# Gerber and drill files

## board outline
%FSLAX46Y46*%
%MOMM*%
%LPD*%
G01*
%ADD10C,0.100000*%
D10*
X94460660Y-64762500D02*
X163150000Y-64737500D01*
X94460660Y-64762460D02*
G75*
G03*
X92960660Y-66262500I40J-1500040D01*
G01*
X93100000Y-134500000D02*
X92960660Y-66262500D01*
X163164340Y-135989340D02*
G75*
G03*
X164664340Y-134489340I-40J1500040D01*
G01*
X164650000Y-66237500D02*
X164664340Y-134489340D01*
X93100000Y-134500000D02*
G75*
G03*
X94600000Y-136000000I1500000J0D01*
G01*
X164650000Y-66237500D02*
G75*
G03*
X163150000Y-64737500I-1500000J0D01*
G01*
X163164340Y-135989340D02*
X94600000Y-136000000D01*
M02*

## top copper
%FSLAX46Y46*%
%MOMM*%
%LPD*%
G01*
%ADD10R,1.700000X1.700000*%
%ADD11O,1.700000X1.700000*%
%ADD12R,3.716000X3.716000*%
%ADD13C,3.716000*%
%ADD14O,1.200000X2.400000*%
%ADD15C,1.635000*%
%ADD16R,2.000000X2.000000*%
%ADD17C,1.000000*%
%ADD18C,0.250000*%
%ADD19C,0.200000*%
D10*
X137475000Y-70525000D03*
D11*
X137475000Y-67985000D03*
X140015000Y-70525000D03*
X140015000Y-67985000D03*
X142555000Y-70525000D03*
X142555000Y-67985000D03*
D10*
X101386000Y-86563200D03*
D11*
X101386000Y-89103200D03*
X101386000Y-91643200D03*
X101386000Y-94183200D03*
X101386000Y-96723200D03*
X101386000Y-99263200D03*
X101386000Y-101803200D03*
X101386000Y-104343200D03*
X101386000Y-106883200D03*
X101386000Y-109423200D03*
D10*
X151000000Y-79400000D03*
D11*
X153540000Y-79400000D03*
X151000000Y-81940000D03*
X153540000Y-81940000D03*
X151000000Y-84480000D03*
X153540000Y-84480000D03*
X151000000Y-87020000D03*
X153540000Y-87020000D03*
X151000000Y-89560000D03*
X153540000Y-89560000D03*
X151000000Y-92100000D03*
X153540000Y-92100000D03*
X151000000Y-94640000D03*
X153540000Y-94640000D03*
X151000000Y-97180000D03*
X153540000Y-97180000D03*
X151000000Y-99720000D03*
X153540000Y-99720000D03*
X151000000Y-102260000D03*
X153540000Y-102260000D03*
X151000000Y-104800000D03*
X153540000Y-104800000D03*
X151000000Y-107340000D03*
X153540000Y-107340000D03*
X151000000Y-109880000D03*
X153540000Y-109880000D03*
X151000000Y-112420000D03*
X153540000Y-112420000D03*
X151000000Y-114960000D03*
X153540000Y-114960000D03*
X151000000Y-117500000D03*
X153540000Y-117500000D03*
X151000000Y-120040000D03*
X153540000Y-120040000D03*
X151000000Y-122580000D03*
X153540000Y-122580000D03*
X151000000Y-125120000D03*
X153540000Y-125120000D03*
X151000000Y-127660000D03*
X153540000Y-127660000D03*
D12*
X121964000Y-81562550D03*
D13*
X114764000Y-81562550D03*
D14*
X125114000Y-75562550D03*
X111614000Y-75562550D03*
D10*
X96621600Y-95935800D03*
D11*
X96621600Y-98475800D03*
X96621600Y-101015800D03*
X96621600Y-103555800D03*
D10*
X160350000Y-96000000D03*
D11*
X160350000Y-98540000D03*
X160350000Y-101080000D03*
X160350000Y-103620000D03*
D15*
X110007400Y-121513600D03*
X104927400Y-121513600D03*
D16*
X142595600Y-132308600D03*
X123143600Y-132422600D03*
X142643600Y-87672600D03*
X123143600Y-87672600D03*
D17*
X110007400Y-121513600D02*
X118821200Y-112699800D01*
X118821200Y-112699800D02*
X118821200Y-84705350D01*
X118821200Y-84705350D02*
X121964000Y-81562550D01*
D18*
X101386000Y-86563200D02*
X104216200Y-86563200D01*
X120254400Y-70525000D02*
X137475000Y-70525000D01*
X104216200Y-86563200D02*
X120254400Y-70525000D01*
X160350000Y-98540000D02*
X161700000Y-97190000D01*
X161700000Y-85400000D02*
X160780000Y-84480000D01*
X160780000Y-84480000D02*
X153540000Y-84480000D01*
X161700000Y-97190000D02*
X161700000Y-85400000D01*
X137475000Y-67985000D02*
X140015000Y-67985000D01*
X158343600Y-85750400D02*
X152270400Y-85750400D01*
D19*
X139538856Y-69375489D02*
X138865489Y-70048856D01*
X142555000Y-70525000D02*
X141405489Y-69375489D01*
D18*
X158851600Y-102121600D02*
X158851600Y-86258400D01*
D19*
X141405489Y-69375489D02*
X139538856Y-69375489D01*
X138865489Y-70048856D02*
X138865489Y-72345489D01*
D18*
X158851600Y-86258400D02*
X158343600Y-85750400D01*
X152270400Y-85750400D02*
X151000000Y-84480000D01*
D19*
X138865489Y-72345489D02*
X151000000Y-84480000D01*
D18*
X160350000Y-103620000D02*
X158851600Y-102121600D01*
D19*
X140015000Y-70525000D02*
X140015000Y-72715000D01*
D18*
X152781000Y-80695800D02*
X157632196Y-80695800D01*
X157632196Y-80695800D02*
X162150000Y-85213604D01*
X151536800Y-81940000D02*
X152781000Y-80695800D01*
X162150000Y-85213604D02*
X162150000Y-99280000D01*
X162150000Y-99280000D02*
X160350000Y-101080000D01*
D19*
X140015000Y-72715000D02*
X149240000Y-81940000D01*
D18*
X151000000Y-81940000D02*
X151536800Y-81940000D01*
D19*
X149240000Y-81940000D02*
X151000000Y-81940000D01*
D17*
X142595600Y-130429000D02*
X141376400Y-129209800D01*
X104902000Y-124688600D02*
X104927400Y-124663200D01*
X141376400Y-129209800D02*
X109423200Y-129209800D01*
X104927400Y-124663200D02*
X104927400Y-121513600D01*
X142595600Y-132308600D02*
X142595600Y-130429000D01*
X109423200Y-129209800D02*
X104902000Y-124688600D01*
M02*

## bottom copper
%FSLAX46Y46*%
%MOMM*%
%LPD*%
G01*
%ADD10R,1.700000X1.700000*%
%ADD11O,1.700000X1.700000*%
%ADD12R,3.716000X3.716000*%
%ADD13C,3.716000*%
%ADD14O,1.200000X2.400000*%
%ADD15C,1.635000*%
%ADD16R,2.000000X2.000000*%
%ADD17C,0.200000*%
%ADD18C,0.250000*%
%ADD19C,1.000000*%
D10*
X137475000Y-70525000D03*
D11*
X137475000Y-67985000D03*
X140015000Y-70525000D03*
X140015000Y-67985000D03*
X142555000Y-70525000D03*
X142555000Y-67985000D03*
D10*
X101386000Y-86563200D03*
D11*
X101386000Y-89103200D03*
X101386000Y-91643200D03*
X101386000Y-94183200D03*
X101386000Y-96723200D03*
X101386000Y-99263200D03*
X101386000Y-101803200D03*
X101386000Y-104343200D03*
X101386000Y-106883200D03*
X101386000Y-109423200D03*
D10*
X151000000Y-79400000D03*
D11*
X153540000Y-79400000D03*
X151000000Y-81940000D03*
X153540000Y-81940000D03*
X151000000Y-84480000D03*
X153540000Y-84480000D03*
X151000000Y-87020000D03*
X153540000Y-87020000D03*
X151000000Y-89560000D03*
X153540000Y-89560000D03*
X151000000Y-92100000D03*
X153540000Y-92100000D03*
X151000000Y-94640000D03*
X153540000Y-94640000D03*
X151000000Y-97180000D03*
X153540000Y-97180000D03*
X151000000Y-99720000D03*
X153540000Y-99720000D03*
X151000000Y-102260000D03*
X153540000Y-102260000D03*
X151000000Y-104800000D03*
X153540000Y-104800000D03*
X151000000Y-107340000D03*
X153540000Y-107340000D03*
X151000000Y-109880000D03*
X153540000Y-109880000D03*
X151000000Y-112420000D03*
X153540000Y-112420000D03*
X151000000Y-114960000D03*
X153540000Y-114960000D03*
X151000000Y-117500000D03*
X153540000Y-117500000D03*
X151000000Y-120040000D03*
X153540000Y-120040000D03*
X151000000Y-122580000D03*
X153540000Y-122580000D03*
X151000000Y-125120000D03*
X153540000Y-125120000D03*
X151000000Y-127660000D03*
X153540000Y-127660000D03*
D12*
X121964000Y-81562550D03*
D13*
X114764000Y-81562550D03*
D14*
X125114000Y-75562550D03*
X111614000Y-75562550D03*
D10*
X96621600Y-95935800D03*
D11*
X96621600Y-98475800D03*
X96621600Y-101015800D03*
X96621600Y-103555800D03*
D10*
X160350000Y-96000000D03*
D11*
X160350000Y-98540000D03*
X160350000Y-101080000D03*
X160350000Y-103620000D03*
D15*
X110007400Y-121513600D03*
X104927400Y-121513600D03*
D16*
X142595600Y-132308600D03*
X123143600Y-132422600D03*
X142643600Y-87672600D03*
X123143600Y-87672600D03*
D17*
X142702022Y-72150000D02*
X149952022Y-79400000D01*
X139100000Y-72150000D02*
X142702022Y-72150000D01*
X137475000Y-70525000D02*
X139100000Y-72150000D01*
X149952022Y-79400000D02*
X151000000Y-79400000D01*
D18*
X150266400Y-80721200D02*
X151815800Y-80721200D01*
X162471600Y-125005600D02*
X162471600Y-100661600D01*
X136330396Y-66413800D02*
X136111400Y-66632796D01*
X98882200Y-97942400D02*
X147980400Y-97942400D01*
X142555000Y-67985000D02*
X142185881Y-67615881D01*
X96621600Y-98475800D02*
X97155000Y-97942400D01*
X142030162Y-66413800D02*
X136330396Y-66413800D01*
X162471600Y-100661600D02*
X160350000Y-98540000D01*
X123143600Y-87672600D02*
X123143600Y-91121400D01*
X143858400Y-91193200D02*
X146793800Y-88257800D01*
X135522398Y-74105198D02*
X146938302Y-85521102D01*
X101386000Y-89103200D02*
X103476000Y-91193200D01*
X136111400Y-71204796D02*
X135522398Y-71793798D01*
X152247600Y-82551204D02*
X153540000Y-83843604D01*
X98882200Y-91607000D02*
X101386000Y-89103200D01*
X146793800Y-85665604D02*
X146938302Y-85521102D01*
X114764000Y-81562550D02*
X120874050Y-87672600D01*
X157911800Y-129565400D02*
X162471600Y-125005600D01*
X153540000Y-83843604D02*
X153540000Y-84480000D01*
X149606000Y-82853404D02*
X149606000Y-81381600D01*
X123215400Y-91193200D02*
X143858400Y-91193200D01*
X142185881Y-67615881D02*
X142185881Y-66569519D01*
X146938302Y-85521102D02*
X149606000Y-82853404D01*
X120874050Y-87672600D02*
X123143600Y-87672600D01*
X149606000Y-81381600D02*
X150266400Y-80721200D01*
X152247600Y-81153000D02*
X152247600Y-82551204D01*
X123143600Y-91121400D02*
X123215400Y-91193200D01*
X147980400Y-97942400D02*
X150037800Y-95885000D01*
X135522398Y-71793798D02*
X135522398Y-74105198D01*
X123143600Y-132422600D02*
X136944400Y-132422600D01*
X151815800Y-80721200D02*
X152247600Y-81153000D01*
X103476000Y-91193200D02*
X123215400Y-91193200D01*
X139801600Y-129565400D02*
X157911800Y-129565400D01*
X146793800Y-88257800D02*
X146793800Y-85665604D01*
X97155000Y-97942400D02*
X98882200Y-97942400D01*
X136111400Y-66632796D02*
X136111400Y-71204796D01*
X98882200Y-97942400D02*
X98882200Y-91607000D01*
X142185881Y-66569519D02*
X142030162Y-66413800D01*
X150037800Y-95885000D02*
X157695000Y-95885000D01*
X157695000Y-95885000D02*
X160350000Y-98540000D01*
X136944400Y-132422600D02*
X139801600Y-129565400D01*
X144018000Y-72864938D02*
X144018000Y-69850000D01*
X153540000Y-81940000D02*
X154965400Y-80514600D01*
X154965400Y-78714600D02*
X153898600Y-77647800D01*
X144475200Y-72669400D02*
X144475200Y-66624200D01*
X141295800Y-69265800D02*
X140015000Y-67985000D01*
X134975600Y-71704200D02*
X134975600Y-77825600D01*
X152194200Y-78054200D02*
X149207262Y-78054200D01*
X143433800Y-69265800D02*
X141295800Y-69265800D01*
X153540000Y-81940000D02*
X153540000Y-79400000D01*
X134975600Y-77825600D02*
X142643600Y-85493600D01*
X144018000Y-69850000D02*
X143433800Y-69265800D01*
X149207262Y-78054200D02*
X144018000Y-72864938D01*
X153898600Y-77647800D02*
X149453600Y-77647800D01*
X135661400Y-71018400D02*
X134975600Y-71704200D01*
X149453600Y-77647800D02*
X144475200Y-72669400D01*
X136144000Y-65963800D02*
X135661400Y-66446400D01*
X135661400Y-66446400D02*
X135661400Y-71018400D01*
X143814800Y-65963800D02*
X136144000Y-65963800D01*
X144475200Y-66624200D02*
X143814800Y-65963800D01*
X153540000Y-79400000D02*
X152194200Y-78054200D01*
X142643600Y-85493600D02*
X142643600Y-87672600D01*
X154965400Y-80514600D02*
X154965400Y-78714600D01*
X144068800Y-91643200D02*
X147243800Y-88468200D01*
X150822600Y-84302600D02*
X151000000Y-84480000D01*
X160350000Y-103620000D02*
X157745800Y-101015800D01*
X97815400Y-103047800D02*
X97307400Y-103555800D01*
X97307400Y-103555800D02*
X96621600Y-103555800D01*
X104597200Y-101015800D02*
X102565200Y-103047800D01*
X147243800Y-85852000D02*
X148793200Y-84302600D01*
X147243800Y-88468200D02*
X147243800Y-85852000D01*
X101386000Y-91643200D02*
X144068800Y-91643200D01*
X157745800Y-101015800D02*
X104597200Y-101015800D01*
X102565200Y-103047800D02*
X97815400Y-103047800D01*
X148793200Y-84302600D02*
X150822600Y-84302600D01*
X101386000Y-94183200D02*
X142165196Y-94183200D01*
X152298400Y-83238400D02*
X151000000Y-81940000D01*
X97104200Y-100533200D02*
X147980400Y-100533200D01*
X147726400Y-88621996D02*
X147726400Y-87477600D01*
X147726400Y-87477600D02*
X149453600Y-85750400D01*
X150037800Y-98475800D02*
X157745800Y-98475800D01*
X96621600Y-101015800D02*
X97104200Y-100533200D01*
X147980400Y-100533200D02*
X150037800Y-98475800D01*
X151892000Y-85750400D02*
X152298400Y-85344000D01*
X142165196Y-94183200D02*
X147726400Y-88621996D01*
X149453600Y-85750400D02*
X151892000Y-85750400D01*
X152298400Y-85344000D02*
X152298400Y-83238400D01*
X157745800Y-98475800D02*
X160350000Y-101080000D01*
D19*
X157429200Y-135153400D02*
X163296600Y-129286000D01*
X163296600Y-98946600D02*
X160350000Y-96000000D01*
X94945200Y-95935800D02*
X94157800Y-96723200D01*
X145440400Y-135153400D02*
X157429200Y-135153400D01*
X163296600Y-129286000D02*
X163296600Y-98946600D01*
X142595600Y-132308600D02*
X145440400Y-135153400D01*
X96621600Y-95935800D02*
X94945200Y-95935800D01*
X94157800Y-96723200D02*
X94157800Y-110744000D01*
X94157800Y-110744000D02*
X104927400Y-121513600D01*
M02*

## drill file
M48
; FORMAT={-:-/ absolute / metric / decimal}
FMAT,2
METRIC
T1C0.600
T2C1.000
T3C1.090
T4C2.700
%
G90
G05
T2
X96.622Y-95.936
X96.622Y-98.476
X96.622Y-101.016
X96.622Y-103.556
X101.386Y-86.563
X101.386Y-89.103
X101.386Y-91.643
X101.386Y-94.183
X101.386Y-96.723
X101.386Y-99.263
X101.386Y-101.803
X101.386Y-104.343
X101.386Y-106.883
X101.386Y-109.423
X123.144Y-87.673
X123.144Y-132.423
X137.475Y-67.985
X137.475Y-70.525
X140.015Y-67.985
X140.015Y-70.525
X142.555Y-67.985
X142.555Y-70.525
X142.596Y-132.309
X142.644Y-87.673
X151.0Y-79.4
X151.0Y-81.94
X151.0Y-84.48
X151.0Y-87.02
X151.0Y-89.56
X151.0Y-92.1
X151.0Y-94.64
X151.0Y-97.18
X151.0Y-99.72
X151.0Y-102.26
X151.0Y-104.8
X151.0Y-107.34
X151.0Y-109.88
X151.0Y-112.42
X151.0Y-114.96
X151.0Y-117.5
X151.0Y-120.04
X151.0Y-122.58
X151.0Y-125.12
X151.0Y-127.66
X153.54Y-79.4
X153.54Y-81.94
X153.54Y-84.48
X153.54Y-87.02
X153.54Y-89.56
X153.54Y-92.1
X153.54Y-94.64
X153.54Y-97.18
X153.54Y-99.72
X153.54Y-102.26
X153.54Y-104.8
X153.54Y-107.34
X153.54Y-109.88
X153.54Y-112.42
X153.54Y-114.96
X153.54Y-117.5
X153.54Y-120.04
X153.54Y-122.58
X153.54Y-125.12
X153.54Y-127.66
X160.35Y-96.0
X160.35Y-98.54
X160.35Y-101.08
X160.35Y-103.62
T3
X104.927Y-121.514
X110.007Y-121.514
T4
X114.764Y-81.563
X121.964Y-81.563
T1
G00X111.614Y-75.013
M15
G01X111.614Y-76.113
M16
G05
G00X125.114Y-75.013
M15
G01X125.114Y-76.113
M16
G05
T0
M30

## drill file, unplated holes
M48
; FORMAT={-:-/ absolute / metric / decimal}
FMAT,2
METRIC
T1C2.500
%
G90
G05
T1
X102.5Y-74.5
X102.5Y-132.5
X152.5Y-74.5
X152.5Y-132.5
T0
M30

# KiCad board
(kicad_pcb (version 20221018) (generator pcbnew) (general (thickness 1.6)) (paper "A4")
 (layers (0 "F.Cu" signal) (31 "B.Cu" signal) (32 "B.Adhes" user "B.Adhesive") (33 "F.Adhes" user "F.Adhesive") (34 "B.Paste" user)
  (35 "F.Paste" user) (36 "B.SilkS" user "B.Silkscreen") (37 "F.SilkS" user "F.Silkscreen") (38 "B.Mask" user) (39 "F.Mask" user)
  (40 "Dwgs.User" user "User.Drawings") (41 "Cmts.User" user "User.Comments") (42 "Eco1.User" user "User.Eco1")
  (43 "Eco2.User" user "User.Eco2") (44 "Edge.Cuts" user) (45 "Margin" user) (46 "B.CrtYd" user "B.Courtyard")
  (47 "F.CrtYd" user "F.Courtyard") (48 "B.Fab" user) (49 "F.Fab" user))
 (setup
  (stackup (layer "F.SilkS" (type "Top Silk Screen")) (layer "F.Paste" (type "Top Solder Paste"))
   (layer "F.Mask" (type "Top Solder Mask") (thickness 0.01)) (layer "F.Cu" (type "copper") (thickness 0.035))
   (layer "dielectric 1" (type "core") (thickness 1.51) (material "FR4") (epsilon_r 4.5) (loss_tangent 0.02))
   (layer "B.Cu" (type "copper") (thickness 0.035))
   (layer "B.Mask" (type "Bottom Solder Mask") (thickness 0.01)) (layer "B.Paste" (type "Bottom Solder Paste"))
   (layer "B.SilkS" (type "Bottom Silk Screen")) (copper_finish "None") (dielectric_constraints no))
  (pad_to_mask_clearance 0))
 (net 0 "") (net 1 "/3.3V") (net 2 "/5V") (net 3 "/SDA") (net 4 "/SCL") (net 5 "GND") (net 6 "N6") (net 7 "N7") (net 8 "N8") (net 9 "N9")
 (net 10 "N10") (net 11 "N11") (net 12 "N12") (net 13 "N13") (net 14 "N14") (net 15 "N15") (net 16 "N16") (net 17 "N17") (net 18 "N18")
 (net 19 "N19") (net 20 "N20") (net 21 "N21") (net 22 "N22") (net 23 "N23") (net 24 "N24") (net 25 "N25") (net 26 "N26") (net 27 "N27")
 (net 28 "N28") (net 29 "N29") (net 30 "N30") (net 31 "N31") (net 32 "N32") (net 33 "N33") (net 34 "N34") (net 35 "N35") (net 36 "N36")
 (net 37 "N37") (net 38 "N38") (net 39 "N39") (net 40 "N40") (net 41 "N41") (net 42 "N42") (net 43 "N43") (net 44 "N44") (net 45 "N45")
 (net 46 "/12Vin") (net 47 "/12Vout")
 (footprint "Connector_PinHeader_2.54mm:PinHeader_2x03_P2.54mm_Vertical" (layer "F.Cu") (at 137.475 70.525 90)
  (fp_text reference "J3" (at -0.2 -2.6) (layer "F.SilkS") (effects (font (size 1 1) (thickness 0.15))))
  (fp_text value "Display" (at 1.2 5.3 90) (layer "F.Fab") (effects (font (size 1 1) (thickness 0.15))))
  (pad "1" thru_hole rect (at 0 0 90) (size 1.7 1.7) (drill 1) (layers "*.Cu" "*.Mask") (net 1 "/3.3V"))
  (pad "2" thru_hole oval (at 2.54 0 90) (size 1.7 1.7) (drill 1) (layers "*.Cu" "*.Mask") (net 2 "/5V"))
  (pad "3" thru_hole oval (at 0 2.54 90) (size 1.7 1.7) (drill 1) (layers "*.Cu" "*.Mask") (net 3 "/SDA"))
  (pad "4" thru_hole oval (at 2.54 2.54 90) (size 1.7 1.7) (drill 1) (layers "*.Cu" "*.Mask") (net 2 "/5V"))
  (pad "5" thru_hole oval (at 0 5.08 90) (size 1.7 1.7) (drill 1) (layers "*.Cu" "*.Mask") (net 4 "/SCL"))
  (pad "6" thru_hole oval (at 2.54 5.08 90) (size 1.7 1.7) (drill 1) (layers "*.Cu" "*.Mask") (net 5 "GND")))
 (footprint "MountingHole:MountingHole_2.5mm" (layer "F.Cu") (at 152.5 74.5)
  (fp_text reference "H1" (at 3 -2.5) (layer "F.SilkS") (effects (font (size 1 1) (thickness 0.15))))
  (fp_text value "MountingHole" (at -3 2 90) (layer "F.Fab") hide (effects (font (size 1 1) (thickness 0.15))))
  (pad "" np_thru_hole circle (at 0 0) (size 2.5 2.5) (drill 2.5) (layers "*.Cu" "*.Mask")))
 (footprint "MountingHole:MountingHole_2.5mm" (layer "F.Cu") (at 102.5 74.5)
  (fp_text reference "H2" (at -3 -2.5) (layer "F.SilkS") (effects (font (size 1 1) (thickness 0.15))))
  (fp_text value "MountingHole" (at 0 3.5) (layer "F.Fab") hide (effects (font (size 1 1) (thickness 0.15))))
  (pad "" np_thru_hole circle (at 0 0) (size 2.5 2.5) (drill 2.5) (layers "*.Cu" "*.Mask")))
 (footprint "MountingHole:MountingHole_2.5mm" (layer "F.Cu") (at 102.5 132.5)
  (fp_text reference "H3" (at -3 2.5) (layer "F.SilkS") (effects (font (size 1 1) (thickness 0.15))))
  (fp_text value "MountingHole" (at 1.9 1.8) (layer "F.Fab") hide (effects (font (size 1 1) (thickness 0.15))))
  (pad "" np_thru_hole circle (at 0 0) (size 2.5 2.5) (drill 2.5) (layers "*.Cu" "*.Mask")))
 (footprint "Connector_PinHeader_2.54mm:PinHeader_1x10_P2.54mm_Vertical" (layer "F.Cu") (at 101.386 86.5632)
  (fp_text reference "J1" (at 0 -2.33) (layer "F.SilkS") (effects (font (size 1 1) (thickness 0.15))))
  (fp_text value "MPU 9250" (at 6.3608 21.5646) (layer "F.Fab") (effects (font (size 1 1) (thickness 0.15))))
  (pad "1" thru_hole rect (at 0 0) (size 1.7 1.7) (drill 1) (layers "*.Cu" "*.Mask") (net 1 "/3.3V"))
  (pad "2" thru_hole oval (at 0 2.54) (size 1.7 1.7) (drill 1) (layers "*.Cu" "*.Mask") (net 5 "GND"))
  (pad "3" thru_hole oval (at 0 5.08) (size 1.7 1.7) (drill 1) (layers "*.Cu" "*.Mask") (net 4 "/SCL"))
  (pad "4" thru_hole oval (at 0 7.62) (size 1.7 1.7) (drill 1) (layers "*.Cu" "*.Mask") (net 3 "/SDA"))
  (pad "5" thru_hole oval (at 0 10.16) (size 1.7 1.7) (drill 1) (layers "*.Cu" "*.Mask") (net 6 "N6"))
  (pad "6" thru_hole oval (at 0 12.7) (size 1.7 1.7) (drill 1) (layers "*.Cu" "*.Mask") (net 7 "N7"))
  (pad "7" thru_hole oval (at 0 15.24) (size 1.7 1.7) (drill 1) (layers "*.Cu" "*.Mask") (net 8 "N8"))
  (pad "8" thru_hole oval (at 0 17.78) (size 1.7 1.7) (drill 1) (layers "*.Cu" "*.Mask") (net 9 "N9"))
  (pad "9" thru_hole oval (at 0 20.32) (size 1.7 1.7) (drill 1) (layers "*.Cu" "*.Mask") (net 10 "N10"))
  (pad "10" thru_hole oval (at 0 22.86) (size 1.7 1.7) (drill 1) (layers "*.Cu" "*.Mask") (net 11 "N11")))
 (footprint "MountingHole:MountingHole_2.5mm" (layer "F.Cu") (at 152.5 132.5)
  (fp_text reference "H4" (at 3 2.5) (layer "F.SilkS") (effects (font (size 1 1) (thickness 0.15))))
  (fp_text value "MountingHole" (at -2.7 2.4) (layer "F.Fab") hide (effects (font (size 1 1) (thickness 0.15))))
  (pad "" np_thru_hole circle (at 0 0) (size 2.5 2.5) (drill 2.5) (layers "*.Cu" "*.Mask")))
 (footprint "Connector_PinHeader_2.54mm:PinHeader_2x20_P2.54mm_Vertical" (layer "F.Cu") (at 151 79.4)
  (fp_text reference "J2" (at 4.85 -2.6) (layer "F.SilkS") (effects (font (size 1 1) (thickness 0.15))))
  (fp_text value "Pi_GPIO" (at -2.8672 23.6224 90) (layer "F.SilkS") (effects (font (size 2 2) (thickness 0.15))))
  (pad "1" thru_hole rect (at 0 0) (size 1.7 1.7) (drill 1) (layers "*.Cu" "*.Mask") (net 1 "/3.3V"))
  (pad "2" thru_hole oval (at 2.54 0) (size 1.7 1.7) (drill 1) (layers "*.Cu" "*.Mask") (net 2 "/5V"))
  (pad "3" thru_hole oval (at 0 2.54) (size 1.7 1.7) (drill 1) (layers "*.Cu" "*.Mask") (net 3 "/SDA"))
  (pad "4" thru_hole oval (at 2.54 2.54) (size 1.7 1.7) (drill 1) (layers "*.Cu" "*.Mask") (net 2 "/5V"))
  (pad "5" thru_hole oval (at 0 5.08) (size 1.7 1.7) (drill 1) (layers "*.Cu" "*.Mask") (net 4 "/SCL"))
  (pad "6" thru_hole oval (at 2.54 5.08) (size 1.7 1.7) (drill 1) (layers "*.Cu" "*.Mask") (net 5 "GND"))
  (pad "7" thru_hole oval (at 0 7.62) (size 1.7 1.7) (drill 1) (layers "*.Cu" "*.Mask") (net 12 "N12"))
  (pad "8" thru_hole oval (at 2.54 7.62) (size 1.7 1.7) (drill 1) (layers "*.Cu" "*.Mask") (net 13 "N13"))
  (pad "9" thru_hole oval (at 0 10.16) (size 1.7 1.7) (drill 1) (layers "*.Cu" "*.Mask") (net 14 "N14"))
  (pad "10" thru_hole oval (at 2.54 10.16) (size 1.7 1.7) (drill 1) (layers "*.Cu" "*.Mask") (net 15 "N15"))
  (pad "11" thru_hole oval (at 0 12.7) (size 1.7 1.7) (drill 1) (layers "*.Cu" "*.Mask") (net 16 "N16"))
  (pad "12" thru_hole oval (at 2.54 12.7) (size 1.7 1.7) (drill 1) (layers "*.Cu" "*.Mask") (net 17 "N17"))
  (pad "13" thru_hole oval (at 0 15.24) (size 1.7 1.7) (drill 1) (layers "*.Cu" "*.Mask") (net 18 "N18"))
  (pad "14" thru_hole oval (at 2.54 15.24) (size 1.7 1.7) (drill 1) (layers "*.Cu" "*.Mask") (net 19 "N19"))
  (pad "15" thru_hole oval (at 0 17.78) (size 1.7 1.7) (drill 1) (layers "*.Cu" "*.Mask") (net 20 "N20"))
  (pad "16" thru_hole oval (at 2.54 17.78) (size 1.7 1.7) (drill 1) (layers "*.Cu" "*.Mask") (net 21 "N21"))
  (pad "17" thru_hole oval (at 0 20.32) (size 1.7 1.7) (drill 1) (layers "*.Cu" "*.Mask") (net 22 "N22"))
  (pad "18" thru_hole oval (at 2.54 20.32) (size 1.7 1.7) (drill 1) (layers "*.Cu" "*.Mask") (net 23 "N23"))
  (pad "19" thru_hole oval (at 0 22.86) (size 1.7 1.7) (drill 1) (layers "*.Cu" "*.Mask") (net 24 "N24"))
  (pad "20" thru_hole oval (at 2.54 22.86) (size 1.7 1.7) (drill 1) (layers "*.Cu" "*.Mask") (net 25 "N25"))
  (pad "21" thru_hole oval (at 0 25.4) (size 1.7 1.7) (drill 1) (layers "*.Cu" "*.Mask") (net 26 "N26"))
  (pad "22" thru_hole oval (at 2.54 25.4) (size 1.7 1.7) (drill 1) (layers "*.Cu" "*.Mask") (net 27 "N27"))
  (pad "23" thru_hole oval (at 0 27.94) (size 1.7 1.7) (drill 1) (layers "*.Cu" "*.Mask") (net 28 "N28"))
  (pad "24" thru_hole oval (at 2.54 27.94) (size 1.7 1.7) (drill 1) (layers "*.Cu" "*.Mask") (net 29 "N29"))
  (pad "25" thru_hole oval (at 0 30.48) (size 1.7 1.7) (drill 1) (layers "*.Cu" "*.Mask") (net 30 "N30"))
  (pad "26" thru_hole oval (at 2.54 30.48) (size 1.7 1.7) (drill 1) (layers "*.Cu" "*.Mask") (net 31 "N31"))
  (pad "27" thru_hole oval (at 0 33.02) (size 1.7 1.7) (drill 1) (layers "*.Cu" "*.Mask") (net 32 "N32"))
  (pad "28" thru_hole oval (at 2.54 33.02) (size 1.7 1.7) (drill 1) (layers "*.Cu" "*.Mask") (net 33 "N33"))
  (pad "29" thru_hole oval (at 0 35.56) (size 1.7 1.7) (drill 1) (layers "*.Cu" "*.Mask") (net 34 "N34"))
  (pad "30" thru_hole oval (at 2.54 35.56) (size 1.7 1.7) (drill 1) (layers "*.Cu" "*.Mask") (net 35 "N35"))
  (pad "31" thru_hole oval (at 0 38.1) (size 1.7 1.7) (drill 1) (layers "*.Cu" "*.Mask") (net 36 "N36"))
  (pad "32" thru_hole oval (at 2.54 38.1) (size 1.7 1.7) (drill 1) (layers "*.Cu" "*.Mask") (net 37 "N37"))
  (pad "33" thru_hole oval (at 0 40.64) (size 1.7 1.7) (drill 1) (layers "*.Cu" "*.Mask") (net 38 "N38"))
  (pad "34" thru_hole oval (at 2.54 40.64) (size 1.7 1.7) (drill 1) (layers "*.Cu" "*.Mask") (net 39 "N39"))
  (pad "35" thru_hole oval (at 0 43.18) (size 1.7 1.7) (drill 1) (layers "*.Cu" "*.Mask") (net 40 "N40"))
  (pad "36" thru_hole oval (at 2.54 43.18) (size 1.7 1.7) (drill 1) (layers "*.Cu" "*.Mask") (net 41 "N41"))
  (pad "37" thru_hole oval (at 0 45.72) (size 1.7 1.7) (drill 1) (layers "*.Cu" "*.Mask") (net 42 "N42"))
  (pad "38" thru_hole oval (at 2.54 45.72) (size 1.7 1.7) (drill 1) (layers "*.Cu" "*.Mask") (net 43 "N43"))
  (pad "39" thru_hole oval (at 0 48.26) (size 1.7 1.7) (drill 1) (layers "*.Cu" "*.Mask") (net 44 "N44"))
  (pad "40" thru_hole oval (at 2.54 48.26) (size 1.7 1.7) (drill 1) (layers "*.Cu" "*.Mask") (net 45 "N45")))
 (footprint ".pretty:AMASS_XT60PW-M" (layer "F.Cu") (at 118.364 75.56255)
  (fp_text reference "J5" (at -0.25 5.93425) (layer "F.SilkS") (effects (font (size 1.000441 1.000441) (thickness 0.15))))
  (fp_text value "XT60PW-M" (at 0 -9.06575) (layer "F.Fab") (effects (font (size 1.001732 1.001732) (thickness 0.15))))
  (pad "1" thru_hole rect (at 3.6 6) (size 3.716 3.716) (drill 2.7) (layers "*.Cu" "*.Mask") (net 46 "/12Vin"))
  (pad "2" thru_hole circle (at -3.6 6) (size 3.716 3.716) (drill 2.7) (layers "*.Cu" "*.Mask") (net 5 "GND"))
  (pad "S1" thru_hole oval (at 6.75 0) (size 1.2 2.4) (drill oval 0.6 1.7) (layers "*.Cu" "*.Mask"))
  (pad "S2" thru_hole oval (at -6.75 0) (size 1.2 2.4) (drill oval 0.6 1.7) (layers "*.Cu" "*.Mask")))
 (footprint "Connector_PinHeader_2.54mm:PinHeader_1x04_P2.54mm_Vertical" (layer "F.Cu") (at 96.6216 95.9358)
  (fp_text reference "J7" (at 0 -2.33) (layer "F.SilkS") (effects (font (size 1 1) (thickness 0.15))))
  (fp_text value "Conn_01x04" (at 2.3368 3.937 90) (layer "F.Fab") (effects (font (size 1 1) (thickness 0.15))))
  (pad "1" thru_hole rect (at 0 0) (size 1.7 1.7) (drill 1) (layers "*.Cu" "*.Mask") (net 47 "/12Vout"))
  (pad "2" thru_hole oval (at 0 2.54) (size 1.7 1.7) (drill 1) (layers "*.Cu" "*.Mask") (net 5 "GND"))
  (pad "3" thru_hole oval (at 0 5.08) (size 1.7 1.7) (drill 1) (layers "*.Cu" "*.Mask") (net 3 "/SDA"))
  (pad "4" thru_hole oval (at 0 7.62) (size 1.7 1.7) (drill 1) (layers "*.Cu" "*.Mask") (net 4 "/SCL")))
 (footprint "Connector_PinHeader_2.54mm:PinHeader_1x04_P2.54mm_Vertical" (layer "F.Cu") (at 160.35 96)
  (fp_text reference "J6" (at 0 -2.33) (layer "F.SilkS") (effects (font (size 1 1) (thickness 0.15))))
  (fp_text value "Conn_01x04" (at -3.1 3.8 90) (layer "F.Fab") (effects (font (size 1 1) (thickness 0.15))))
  (pad "1" thru_hole rect (at 0 0) (size 1.7 1.7) (drill 1) (layers "*.Cu" "*.Mask") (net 47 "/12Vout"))
  (pad "2" thru_hole oval (at 0 2.54) (size 1.7 1.7) (drill 1) (layers "*.Cu" "*.Mask") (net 5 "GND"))
  (pad "3" thru_hole oval (at 0 5.08) (size 1.7 1.7) (drill 1) (layers "*.Cu" "*.Mask") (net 3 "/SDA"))
  (pad "4" thru_hole oval (at 0 7.62) (size 1.7 1.7) (drill 1) (layers "*.Cu" "*.Mask") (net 4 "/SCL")))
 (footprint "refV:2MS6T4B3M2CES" (layer "F.Cu") (at 110.0074 121.5136 90)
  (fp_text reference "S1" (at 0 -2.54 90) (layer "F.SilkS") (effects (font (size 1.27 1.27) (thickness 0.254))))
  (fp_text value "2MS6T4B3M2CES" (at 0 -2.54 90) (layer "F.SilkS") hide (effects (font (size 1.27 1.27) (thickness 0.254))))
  (pad "1" thru_hole circle (at 0 0 90) (size 1.635 1.635) (drill 1.09) (layers "*.Cu" "*.Mask") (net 46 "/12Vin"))
  (pad "3" thru_hole circle (at 0 -5.08 90) (size 1.635 1.635) (drill 1.09) (layers "*.Cu" "*.Mask") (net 47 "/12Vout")))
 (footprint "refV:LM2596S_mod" (layer "B.Cu") (at 145.6436 123.6726 90)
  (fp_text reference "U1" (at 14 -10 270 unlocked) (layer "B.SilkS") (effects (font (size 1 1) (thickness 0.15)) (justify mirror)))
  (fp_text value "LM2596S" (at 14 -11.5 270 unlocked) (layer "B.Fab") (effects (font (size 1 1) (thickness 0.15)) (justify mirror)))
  (pad "1" thru_hole rect (at -8.636 -3.048 90) (size 2 2) (drill 1) (layers "*.Cu" "*.Mask") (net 47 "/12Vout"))
  (pad "2" thru_hole rect (at -8.75 -22.5 90) (size 2 2) (drill 1) (layers "*.Cu" "*.Mask") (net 5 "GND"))
  (pad "3" thru_hole rect (at 36 -3 90) (size 2 2) (drill 1) (layers "*.Cu" "*.Mask") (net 2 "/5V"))
  (pad "4" thru_hole rect (at 36 -22.5 90) (size 2 2) (drill 1) (layers "*.Cu" "*.Mask") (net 5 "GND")))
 (gr_line (start 94.46066 64.7625) (end 163.15 64.7375) (stroke (width 0.1) (type solid)) (layer "Edge.Cuts"))
 (gr_arc (start 92.96066 66.2625) (mid 93.400012 65.201852) (end 94.46066 64.7625) (stroke (width 0.1) (type solid)) (layer "Edge.Cuts"))
 (gr_line (start 93.1 134.5) (end 92.96066 66.2625) (stroke (width 0.1) (type solid)) (layer "Edge.Cuts"))
 (gr_arc (start 164.66434 134.48934) (mid 164.225 135.55) (end 163.16434 135.98934) (stroke (width 0.1) (type solid)) (layer "Edge.Cuts"))
 (gr_line (start 164.65 66.2375) (end 164.66434 134.48934) (stroke (width 0.1) (type solid)) (layer "Edge.Cuts"))
 (gr_arc (start 94.6 136) (mid 93.53934 135.56066) (end 93.1 134.5) (stroke (width 0.1) (type solid)) (layer "Edge.Cuts"))
 (gr_arc (start 163.15 64.7375) (mid 164.210674 65.176837) (end 164.65 66.2375) (stroke (width 0.1) (type solid)) (layer "Edge.Cuts"))
 (gr_line (start 163.16434 135.98934) (end 94.6 136) (stroke (width 0.1) (type solid)) (layer "Edge.Cuts"))
 (segment (start 110.0074 121.5136) (end 118.8212 112.6998) (width 1) (layer "F.Cu") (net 46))
 (segment (start 118.8212 112.6998) (end 118.8212 84.70535) (width 1) (layer "F.Cu") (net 46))
 (segment (start 118.8212 84.70535) (end 121.964 81.56255) (width 1) (layer "F.Cu") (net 46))
 (segment (start 101.386 86.5632) (end 104.2162 86.5632) (width 0.25) (layer "F.Cu") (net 1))
 (segment (start 120.2544 70.525) (end 137.475 70.525) (width 0.25) (layer "F.Cu") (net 1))
 (segment (start 104.2162 86.5632) (end 120.2544 70.525) (width 0.25) (layer "F.Cu") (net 1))
 (segment (start 142.702022 72.15) (end 149.952022 79.4) (width 0.2) (layer "B.Cu") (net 1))
 (segment (start 139.1 72.15) (end 142.702022 72.15) (width 0.2) (layer "B.Cu") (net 1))
 (segment (start 137.475 70.525) (end 139.1 72.15) (width 0.2) (layer "B.Cu") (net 1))
 (segment (start 149.952022 79.4) (end 151 79.4) (width 0.2) (layer "B.Cu") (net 1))
 (segment (start 160.35 98.54) (end 161.7 97.19) (width 0.25) (layer "F.Cu") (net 5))
 (segment (start 161.7 85.4) (end 160.78 84.48) (width 0.25) (layer "F.Cu") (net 5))
 (segment (start 160.78 84.48) (end 153.54 84.48) (width 0.25) (layer "F.Cu") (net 5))
 (segment (start 161.7 97.19) (end 161.7 85.4) (width 0.25) (layer "F.Cu") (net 5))
 (segment (start 150.2664 80.7212) (end 151.8158 80.7212) (width 0.25) (layer "B.Cu") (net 5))
 (segment (start 162.4716 125.0056) (end 162.4716 100.6616) (width 0.25) (layer "B.Cu") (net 5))
 (segment (start 136.330396 66.4138) (end 136.1114 66.632796) (width 0.25) (layer "B.Cu") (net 5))
 (segment (start 98.8822 97.9424) (end 147.9804 97.9424) (width 0.25) (layer "B.Cu") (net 5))
 (segment (start 142.555 67.985) (end 142.185881 67.615881) (width 0.25) (layer "B.Cu") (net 5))
 (segment (start 96.6216 98.4758) (end 97.155 97.9424) (width 0.25) (layer "B.Cu") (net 5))
 (segment (start 142.030162 66.4138) (end 136.330396 66.4138) (width 0.25) (layer "B.Cu") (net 5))
 (segment (start 162.4716 100.6616) (end 160.35 98.54) (width 0.25) (layer "B.Cu") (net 5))
 (segment (start 123.1436 87.6726) (end 123.1436 91.1214) (width 0.25) (layer "B.Cu") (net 5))
 (segment (start 143.8584 91.1932) (end 146.7938 88.2578) (width 0.25) (layer "B.Cu") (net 5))
 (segment (start 135.522398 74.105198) (end 146.938302 85.521102) (width 0.25) (layer "B.Cu") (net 5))
 (segment (start 101.386 89.1032) (end 103.476 91.1932) (width 0.25) (layer "B.Cu") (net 5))
 (segment (start 136.1114 71.204796) (end 135.522398 71.793798) (width 0.25) (layer "B.Cu") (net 5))
 (segment (start 152.2476 82.551204) (end 153.54 83.843604) (width 0.25) (layer "B.Cu") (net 5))
 (segment (start 98.8822 91.607) (end 101.386 89.1032) (width 0.25) (layer "B.Cu") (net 5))
 (segment (start 146.7938 85.665604) (end 146.938302 85.521102) (width 0.25) (layer "B.Cu") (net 5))
 (segment (start 114.764 81.56255) (end 120.87405 87.6726) (width 0.25) (layer "B.Cu") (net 5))
 (segment (start 157.9118 129.5654) (end 162.4716 125.0056) (width 0.25) (layer "B.Cu") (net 5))
 (segment (start 153.54 83.843604) (end 153.54 84.48) (width 0.25) (layer "B.Cu") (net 5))
 (segment (start 149.606 82.853404) (end 149.606 81.3816) (width 0.25) (layer "B.Cu") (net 5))
 (segment (start 123.2154 91.1932) (end 143.8584 91.1932) (width 0.25) (layer "B.Cu") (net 5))
 (segment (start 142.185881 67.615881) (end 142.185881 66.569519) (width 0.25) (layer "B.Cu") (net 5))
 (segment (start 146.938302 85.521102) (end 149.606 82.853404) (width 0.25) (layer "B.Cu") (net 5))
 (segment (start 120.87405 87.6726) (end 123.1436 87.6726) (width 0.25) (layer "B.Cu") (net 5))
 (segment (start 149.606 81.3816) (end 150.2664 80.7212) (width 0.25) (layer "B.Cu") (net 5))
 (segment (start 152.2476 81.153) (end 152.2476 82.551204) (width 0.25) (layer "B.Cu") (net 5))
 (segment (start 123.1436 91.1214) (end 123.2154 91.1932) (width 0.25) (layer "B.Cu") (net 5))
 (segment (start 147.9804 97.9424) (end 150.0378 95.885) (width 0.25) (layer "B.Cu") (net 5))
 (segment (start 135.522398 71.793798) (end 135.522398 74.105198) (width 0.25) (layer "B.Cu") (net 5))
 (segment (start 123.1436 132.4226) (end 136.9444 132.4226) (width 0.25) (layer "B.Cu") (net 5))
 (segment (start 151.8158 80.7212) (end 152.2476 81.153) (width 0.25) (layer "B.Cu") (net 5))
 (segment (start 103.476 91.1932) (end 123.2154 91.1932) (width 0.25) (layer "B.Cu") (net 5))
 (segment (start 139.8016 129.5654) (end 157.9118 129.5654) (width 0.25) (layer "B.Cu") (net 5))
 (segment (start 146.7938 88.2578) (end 146.7938 85.665604) (width 0.25) (layer "B.Cu") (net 5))
 (segment (start 97.155 97.9424) (end 98.8822 97.9424) (width 0.25) (layer "B.Cu") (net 5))
 (segment (start 136.1114 66.632796) (end 136.1114 71.204796) (width 0.25) (layer "B.Cu") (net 5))
 (segment (start 98.8822 97.9424) (end 98.8822 91.607) (width 0.25) (layer "B.Cu") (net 5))
 (segment (start 142.185881 66.569519) (end 142.030162 66.4138) (width 0.25) (layer "B.Cu") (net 5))
 (segment (start 150.0378 95.885) (end 157.695 95.885) (width 0.25) (layer "B.Cu") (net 5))
 (segment (start 157.695 95.885) (end 160.35 98.54) (width 0.25) (layer "B.Cu") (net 5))
 (segment (start 136.9444 132.4226) (end 139.8016 129.5654) (width 0.25) (layer "B.Cu") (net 5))
 (segment (start 137.475 67.985) (end 140.015 67.985) (width 0.25) (layer "F.Cu") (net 2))
 (segment (start 144.018 72.864938) (end 144.018 69.85) (width 0.25) (layer "B.Cu") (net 2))
 (segment (start 153.54 81.94) (end 154.9654 80.5146) (width 0.25) (layer "B.Cu") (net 2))
 (segment (start 154.9654 78.7146) (end 153.8986 77.6478) (width 0.25) (layer "B.Cu") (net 2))
 (segment (start 144.4752 72.6694) (end 144.4752 66.6242) (width 0.25) (layer "B.Cu") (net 2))
 (segment (start 141.2958 69.2658) (end 140.015 67.985) (width 0.25) (layer "B.Cu") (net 2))
 (segment (start 134.9756 71.7042) (end 134.9756 77.8256) (width 0.25) (layer "B.Cu") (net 2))
 (segment (start 152.1942 78.0542) (end 149.207262 78.0542) (width 0.25) (layer "B.Cu") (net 2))
 (segment (start 143.4338 69.2658) (end 141.2958 69.2658) (width 0.25) (layer "B.Cu") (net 2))
 (segment (start 153.54 81.94) (end 153.54 79.4) (width 0.25) (layer "B.Cu") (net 2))
 (segment (start 134.9756 77.8256) (end 142.6436 85.4936) (width 0.25) (layer "B.Cu") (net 2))
 (segment (start 144.018 69.85) (end 143.4338 69.2658) (width 0.25) (layer "B.Cu") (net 2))
 (segment (start 149.207262 78.0542) (end 144.018 72.864938) (width 0.25) (layer "B.Cu") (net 2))
 (segment (start 153.8986 77.6478) (end 149.4536 77.6478) (width 0.25) (layer "B.Cu") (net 2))
 (segment (start 135.6614 71.0184) (end 134.9756 71.7042) (width 0.25) (layer "B.Cu") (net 2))
 (segment (start 149.4536 77.6478) (end 144.4752 72.6694) (width 0.25) (layer "B.Cu") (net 2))
 (segment (start 136.144 65.9638) (end 135.6614 66.4464) (width 0.25) (layer "B.Cu") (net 2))
 (segment (start 135.6614 66.4464) (end 135.6614 71.0184) (width 0.25) (layer "B.Cu") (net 2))
 (segment (start 143.8148 65.9638) (end 136.144 65.9638) (width 0.25) (layer "B.Cu") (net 2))
 (segment (start 144.4752 66.6242) (end 143.8148 65.9638) (width 0.25) (layer "B.Cu") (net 2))
 (segment (start 153.54 79.4) (end 152.1942 78.0542) (width 0.25) (layer "B.Cu") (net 2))
 (segment (start 142.6436 85.4936) (end 142.6436 87.6726) (width 0.25) (layer "B.Cu") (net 2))
 (segment (start 154.9654 80.5146) (end 154.9654 78.7146) (width 0.25) (layer "B.Cu") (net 2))
 (segment (start 158.3436 85.7504) (end 152.2704 85.7504) (width 0.25) (layer "F.Cu") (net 4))
 (segment (start 139.538856 69.375489) (end 138.865489 70.048856) (width 0.2) (layer "F.Cu") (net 4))
 (segment (start 142.555 70.525) (end 141.405489 69.375489) (width 0.2) (layer "F.Cu") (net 4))
 (segment (start 158.8516 102.1216) (end 158.8516 86.2584) (width 0.25) (layer "F.Cu") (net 4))
 (segment (start 141.405489 69.375489) (end 139.538856 69.375489) (width 0.2) (layer "F.Cu") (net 4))
 (segment (start 138.865489 70.048856) (end 138.865489 72.345489) (width 0.2) (layer "F.Cu") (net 4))
 (segment (start 158.8516 86.2584) (end 158.3436 85.7504) (width 0.25) (layer "F.Cu") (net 4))
 (segment (start 152.2704 85.7504) (end 151 84.48) (width 0.25) (layer "F.Cu") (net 4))
 (segment (start 138.865489 72.345489) (end 151 84.48) (width 0.2) (layer "F.Cu") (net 4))
 (segment (start 160.35 103.62) (end 158.8516 102.1216) (width 0.25) (layer "F.Cu") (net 4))
 (segment (start 144.0688 91.6432) (end 147.2438 88.4682) (width 0.25) (layer "B.Cu") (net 4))
 (segment (start 150.8226 84.3026) (end 151 84.48) (width 0.25) (layer "B.Cu") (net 4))
 (segment (start 160.35 103.62) (end 157.7458 101.0158) (width 0.25) (layer "B.Cu") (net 4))
 (segment (start 97.8154 103.0478) (end 97.3074 103.5558) (width 0.25) (layer "B.Cu") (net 4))
 (segment (start 97.3074 103.5558) (end 96.6216 103.5558) (width 0.25) (layer "B.Cu") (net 4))
 (segment (start 104.5972 101.0158) (end 102.5652 103.0478) (width 0.25) (layer "B.Cu") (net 4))
 (segment (start 147.2438 85.852) (end 148.7932 84.3026) (width 0.25) (layer "B.Cu") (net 4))
 (segment (start 147.2438 88.4682) (end 147.2438 85.852) (width 0.25) (layer "B.Cu") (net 4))
 (segment (start 101.386 91.6432) (end 144.0688 91.6432) (width 0.25) (layer "B.Cu") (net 4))
 (segment (start 157.7458 101.0158) (end 104.5972 101.0158) (width 0.25) (layer "B.Cu") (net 4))
 (segment (start 102.5652 103.0478) (end 97.8154 103.0478) (width 0.25) (layer "B.Cu") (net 4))
 (segment (start 148.7932 84.3026) (end 150.8226 84.3026) (width 0.25) (layer "B.Cu") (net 4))
 (segment (start 140.015 70.525) (end 140.015 72.715) (width 0.2) (layer "F.Cu") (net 3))
 (segment (start 152.781 80.6958) (end 157.632196 80.6958) (width 0.25) (layer "F.Cu") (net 3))
 (segment (start 157.632196 80.6958) (end 162.15 85.213604) (width 0.25) (layer "F.Cu") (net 3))
 (segment (start 151.5368 81.94) (end 152.781 80.6958) (width 0.25) (layer "F.Cu") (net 3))
 (segment (start 162.15 85.213604) (end 162.15 99.28) (width 0.25) (layer "F.Cu") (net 3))
 (segment (start 162.15 99.28) (end 160.35 101.08) (width 0.25) (layer "F.Cu") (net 3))
 (segment (start 140.015 72.715) (end 149.24 81.94) (width 0.2) (layer "F.Cu") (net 3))
 (segment (start 151 81.94) (end 151.5368 81.94) (width 0.25) (layer "F.Cu") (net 3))
 (segment (start 149.24 81.94) (end 151 81.94) (width 0.2) (layer "F.Cu") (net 3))
 (segment (start 101.386 94.1832) (end 142.165196 94.1832) (width 0.25) (layer "B.Cu") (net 3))
 (segment (start 152.2984 83.2384) (end 151 81.94) (width 0.25) (layer "B.Cu") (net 3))
 (segment (start 97.1042 100.5332) (end 147.9804 100.5332) (width 0.25) (layer "B.Cu") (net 3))
 (segment (start 147.7264 88.621996) (end 147.7264 87.4776) (width 0.25) (layer "B.Cu") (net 3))
 (segment (start 147.7264 87.4776) (end 149.4536 85.7504) (width 0.25) (layer "B.Cu") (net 3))
 (segment (start 150.0378 98.4758) (end 157.7458 98.4758) (width 0.25) (layer "B.Cu") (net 3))
 (segment (start 96.6216 101.0158) (end 97.1042 100.5332) (width 0.25) (layer "B.Cu") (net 3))
 (segment (start 147.9804 100.5332) (end 150.0378 98.4758) (width 0.25) (layer "B.Cu") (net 3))
 (segment (start 151.892 85.7504) (end 152.2984 85.344) (width 0.25) (layer "B.Cu") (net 3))
 (segment (start 142.165196 94.1832) (end 147.7264 88.621996) (width 0.25) (layer "B.Cu") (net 3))
 (segment (start 149.4536 85.7504) (end 151.892 85.7504) (width 0.25) (layer "B.Cu") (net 3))
 (segment (start 152.2984 85.344) (end 152.2984 83.2384) (width 0.25) (layer "B.Cu") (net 3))
 (segment (start 157.7458 98.4758) (end 160.35 101.08) (width 0.25) (layer "B.Cu") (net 3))
 (segment (start 142.5956 130.429) (end 141.3764 129.2098) (width 1) (layer "F.Cu") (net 47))
 (segment (start 104.902 124.6886) (end 104.9274 124.6632) (width 1) (layer "F.Cu") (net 47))
 (segment (start 141.3764 129.2098) (end 109.4232 129.2098) (width 1) (layer "F.Cu") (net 47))
 (segment (start 104.9274 124.6632) (end 104.9274 121.5136) (width 1) (layer "F.Cu") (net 47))
 (segment (start 142.5956 132.3086) (end 142.5956 130.429) (width 1) (layer "F.Cu") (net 47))
 (segment (start 109.4232 129.2098) (end 104.902 124.6886) (width 1) (layer "F.Cu") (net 47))
 (segment (start 157.4292 135.1534) (end 163.2966 129.286) (width 1) (layer "B.Cu") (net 47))
 (segment (start 163.2966 98.9466) (end 160.35 96) (width 1) (layer "B.Cu") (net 47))
 (segment (start 94.9452 95.9358) (end 94.1578 96.7232) (width 1) (layer "B.Cu") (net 47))
 (segment (start 145.4404 135.1534) (end 157.4292 135.1534) (width 1) (layer "B.Cu") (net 47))
 (segment (start 163.2966 129.286) (end 163.2966 98.9466) (width 1) (layer "B.Cu") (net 47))
 (segment (start 142.5956 132.3086) (end 145.4404 135.1534) (width 1) (layer "B.Cu") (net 47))
 (segment (start 96.6216 95.9358) (end 94.9452 95.9358) (width 1) (layer "B.Cu") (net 47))
 (segment (start 94.1578 96.7232) (end 94.1578 110.744) (width 1) (layer "B.Cu") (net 47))
 (segment (start 94.1578 110.744) (end 104.9274 121.5136) (width 1) (layer "B.Cu") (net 47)))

